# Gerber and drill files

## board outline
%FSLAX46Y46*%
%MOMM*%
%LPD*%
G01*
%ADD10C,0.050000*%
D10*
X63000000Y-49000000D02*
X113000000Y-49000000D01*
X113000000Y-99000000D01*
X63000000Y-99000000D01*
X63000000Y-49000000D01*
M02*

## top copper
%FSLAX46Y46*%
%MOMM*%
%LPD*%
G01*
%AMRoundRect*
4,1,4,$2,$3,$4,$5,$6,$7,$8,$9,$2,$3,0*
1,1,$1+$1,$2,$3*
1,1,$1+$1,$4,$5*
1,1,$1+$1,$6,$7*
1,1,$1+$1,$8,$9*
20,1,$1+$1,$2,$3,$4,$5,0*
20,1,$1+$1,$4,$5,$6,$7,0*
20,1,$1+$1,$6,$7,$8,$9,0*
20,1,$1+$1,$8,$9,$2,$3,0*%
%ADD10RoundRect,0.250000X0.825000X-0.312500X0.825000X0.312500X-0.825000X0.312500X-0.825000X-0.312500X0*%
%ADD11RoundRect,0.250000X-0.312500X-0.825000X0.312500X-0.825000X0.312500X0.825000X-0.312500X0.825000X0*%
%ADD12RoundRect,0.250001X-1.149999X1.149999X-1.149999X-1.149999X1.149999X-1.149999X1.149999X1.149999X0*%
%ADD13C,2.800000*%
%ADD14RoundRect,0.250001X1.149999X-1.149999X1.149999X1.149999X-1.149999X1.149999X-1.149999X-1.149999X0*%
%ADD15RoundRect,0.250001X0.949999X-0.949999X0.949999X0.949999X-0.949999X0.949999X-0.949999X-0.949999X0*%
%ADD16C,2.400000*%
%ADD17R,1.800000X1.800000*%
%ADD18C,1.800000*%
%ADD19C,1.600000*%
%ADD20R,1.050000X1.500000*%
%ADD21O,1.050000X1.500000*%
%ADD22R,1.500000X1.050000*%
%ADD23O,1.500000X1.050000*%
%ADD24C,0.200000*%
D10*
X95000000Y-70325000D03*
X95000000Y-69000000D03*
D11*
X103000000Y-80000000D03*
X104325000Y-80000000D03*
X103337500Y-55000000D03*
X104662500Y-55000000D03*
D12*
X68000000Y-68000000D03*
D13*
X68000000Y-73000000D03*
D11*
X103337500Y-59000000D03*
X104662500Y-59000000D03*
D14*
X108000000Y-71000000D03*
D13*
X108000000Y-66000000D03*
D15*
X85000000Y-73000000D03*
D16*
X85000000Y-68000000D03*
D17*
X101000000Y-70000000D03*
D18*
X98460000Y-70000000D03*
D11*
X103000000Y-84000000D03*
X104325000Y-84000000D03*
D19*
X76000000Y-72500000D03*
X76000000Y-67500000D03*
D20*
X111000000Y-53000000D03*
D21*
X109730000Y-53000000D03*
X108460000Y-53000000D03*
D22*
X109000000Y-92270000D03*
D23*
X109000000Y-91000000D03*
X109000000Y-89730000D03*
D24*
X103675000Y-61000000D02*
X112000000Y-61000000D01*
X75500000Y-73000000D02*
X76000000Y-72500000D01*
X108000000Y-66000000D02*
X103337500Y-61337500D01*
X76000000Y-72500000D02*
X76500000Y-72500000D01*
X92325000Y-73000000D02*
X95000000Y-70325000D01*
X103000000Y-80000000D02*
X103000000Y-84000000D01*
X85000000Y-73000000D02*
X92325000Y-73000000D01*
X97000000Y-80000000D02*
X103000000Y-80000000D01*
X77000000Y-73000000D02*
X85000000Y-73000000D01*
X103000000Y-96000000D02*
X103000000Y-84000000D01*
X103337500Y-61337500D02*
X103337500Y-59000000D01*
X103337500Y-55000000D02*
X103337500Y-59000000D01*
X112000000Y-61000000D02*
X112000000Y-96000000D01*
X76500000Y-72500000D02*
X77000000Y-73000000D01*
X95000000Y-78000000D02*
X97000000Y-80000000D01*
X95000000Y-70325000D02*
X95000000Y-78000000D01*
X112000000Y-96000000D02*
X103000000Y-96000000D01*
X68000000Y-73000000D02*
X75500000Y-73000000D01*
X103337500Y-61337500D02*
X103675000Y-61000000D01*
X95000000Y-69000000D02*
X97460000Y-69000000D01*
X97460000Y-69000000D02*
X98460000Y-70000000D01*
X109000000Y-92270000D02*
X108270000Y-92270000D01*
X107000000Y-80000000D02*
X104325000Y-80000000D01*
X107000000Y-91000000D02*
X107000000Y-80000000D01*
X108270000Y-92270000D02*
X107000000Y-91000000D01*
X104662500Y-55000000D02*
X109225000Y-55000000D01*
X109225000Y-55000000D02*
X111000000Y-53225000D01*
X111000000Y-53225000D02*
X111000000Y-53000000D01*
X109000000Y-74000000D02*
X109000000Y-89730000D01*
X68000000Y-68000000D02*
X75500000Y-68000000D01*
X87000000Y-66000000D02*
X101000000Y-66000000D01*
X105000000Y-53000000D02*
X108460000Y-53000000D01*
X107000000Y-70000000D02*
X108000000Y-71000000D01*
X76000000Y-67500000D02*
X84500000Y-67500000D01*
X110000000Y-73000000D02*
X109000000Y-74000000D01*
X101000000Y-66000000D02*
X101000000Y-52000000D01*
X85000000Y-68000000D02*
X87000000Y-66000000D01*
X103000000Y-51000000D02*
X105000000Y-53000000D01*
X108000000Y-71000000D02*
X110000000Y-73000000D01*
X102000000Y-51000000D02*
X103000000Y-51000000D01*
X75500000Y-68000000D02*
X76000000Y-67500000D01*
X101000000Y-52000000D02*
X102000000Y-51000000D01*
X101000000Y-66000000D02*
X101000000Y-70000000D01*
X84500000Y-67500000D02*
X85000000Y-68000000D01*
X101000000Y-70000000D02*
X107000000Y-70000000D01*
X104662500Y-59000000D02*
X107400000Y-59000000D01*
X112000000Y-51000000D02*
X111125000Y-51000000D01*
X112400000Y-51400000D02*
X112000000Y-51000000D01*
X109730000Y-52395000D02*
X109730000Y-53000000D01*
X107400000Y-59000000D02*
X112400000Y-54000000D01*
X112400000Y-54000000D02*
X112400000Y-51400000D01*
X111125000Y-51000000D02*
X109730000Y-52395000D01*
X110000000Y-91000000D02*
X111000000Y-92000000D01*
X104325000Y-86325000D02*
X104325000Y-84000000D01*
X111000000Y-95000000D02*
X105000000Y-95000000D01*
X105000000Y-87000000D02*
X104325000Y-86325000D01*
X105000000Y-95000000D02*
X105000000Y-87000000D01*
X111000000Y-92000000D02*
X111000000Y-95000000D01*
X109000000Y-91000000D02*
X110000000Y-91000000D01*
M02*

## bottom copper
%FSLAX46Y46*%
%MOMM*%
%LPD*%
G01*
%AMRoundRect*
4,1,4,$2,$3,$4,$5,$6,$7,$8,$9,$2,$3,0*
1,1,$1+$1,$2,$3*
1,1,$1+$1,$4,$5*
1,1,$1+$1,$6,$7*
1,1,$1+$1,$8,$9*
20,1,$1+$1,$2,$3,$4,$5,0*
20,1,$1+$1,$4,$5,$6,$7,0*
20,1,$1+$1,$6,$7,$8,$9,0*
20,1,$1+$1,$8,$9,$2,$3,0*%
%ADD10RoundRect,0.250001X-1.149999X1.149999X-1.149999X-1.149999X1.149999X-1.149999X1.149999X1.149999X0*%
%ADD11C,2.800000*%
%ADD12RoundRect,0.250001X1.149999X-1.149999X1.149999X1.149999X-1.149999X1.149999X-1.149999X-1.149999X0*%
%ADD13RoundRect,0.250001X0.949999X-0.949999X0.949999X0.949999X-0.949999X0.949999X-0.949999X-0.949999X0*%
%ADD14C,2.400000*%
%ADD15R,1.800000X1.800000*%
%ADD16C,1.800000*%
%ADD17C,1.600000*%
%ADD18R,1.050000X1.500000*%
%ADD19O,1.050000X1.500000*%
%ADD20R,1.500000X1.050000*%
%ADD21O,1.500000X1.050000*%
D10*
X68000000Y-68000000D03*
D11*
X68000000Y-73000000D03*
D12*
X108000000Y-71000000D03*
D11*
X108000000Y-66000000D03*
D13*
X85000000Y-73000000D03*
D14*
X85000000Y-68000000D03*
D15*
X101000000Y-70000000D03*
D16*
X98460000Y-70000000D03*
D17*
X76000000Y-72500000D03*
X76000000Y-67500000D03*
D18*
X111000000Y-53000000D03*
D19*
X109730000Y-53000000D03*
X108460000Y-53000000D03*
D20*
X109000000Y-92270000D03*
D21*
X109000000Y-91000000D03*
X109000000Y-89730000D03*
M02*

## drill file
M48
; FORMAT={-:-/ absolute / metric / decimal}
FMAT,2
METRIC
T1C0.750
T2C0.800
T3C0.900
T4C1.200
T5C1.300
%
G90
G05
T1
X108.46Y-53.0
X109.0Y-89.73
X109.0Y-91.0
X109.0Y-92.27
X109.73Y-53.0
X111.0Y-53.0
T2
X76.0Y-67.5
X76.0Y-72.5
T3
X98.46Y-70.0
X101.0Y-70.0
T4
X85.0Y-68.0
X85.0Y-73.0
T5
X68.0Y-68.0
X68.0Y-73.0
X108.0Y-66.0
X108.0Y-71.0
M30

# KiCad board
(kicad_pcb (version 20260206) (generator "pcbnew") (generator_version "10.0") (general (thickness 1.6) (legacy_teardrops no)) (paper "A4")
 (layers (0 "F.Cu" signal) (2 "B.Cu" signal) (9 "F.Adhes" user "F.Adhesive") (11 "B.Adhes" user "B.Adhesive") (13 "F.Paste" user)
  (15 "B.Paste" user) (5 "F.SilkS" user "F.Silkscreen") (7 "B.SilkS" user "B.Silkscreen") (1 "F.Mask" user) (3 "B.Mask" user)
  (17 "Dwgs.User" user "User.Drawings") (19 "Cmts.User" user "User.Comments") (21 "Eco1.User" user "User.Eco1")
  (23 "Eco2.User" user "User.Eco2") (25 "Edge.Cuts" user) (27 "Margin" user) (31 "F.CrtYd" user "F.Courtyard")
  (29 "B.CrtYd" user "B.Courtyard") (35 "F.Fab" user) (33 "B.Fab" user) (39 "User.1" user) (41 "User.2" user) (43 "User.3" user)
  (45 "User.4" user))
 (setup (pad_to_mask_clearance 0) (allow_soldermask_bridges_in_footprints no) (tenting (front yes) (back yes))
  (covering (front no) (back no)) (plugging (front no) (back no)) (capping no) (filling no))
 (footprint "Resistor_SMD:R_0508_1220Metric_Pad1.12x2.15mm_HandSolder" (layer "F.Cu") (at 95 69.6625 90)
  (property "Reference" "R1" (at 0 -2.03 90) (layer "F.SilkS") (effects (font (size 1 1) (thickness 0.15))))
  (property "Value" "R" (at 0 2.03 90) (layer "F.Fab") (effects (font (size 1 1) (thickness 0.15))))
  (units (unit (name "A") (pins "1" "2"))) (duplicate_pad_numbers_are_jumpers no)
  (pad "1" smd roundrect (at -0.6625 0 90) (size 1.125 2.15) (layers "F.Cu" "F.Mask" "F.Paste") (roundrect_rratio 0.222222) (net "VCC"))
  (pad "2" smd roundrect (at 0.6625 0 90) (size 1.125 2.15) (layers "F.Cu" "F.Mask" "F.Paste") (roundrect_rratio 0.222222)
   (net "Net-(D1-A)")))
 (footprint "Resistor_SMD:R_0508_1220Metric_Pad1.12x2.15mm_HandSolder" (layer "F.Cu") (at 103.6625 80)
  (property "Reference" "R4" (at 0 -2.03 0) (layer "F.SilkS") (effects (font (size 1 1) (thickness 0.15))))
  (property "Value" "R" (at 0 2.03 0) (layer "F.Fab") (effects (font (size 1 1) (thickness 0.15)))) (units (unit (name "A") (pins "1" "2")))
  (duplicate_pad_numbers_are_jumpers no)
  (pad "1" smd roundrect (at -0.6625 0) (size 1.125 2.15) (layers "F.Cu" "F.Mask" "F.Paste") (roundrect_rratio 0.222222) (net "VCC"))
  (pad "2" smd roundrect (at 0.6625 0) (size 1.125 2.15) (layers "F.Cu" "F.Mask" "F.Paste") (roundrect_rratio 0.222222) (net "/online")))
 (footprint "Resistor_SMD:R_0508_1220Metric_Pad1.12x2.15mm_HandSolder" (layer "F.Cu") (at 104 55)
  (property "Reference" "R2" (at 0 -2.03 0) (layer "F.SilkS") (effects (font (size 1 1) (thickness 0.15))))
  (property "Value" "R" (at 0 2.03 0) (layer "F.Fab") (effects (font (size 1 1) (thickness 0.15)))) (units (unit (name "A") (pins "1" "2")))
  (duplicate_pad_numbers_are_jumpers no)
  (pad "1" smd roundrect (at -0.6625 0) (size 1.125 2.15) (layers "F.Cu" "F.Mask" "F.Paste") (roundrect_rratio 0.222222) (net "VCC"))
  (pad "2" smd roundrect (at 0.6625 0) (size 1.125 2.15) (layers "F.Cu" "F.Mask" "F.Paste") (roundrect_rratio 0.222222) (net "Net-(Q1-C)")))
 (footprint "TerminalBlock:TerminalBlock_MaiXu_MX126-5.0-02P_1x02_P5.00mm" (layer "F.Cu") (at 68 68 -90)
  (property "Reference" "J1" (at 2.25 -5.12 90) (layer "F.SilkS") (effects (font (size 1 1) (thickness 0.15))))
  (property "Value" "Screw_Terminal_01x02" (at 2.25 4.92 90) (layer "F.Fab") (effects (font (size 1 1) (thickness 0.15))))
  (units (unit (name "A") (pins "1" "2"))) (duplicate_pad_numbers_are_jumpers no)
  (pad "1" thru_hole roundrect (at 0 0 270) (size 2.8 2.8) (drill 1.3) (layers "*.Cu" "*.Mask") (remove_unused_layers no)
   (roundrect_rratio 0.089286) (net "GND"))
  (pad "2" thru_hole circle (at 5 0 270) (size 2.8 2.8) (drill 1.3) (layers "*.Cu" "*.Mask") (remove_unused_layers no) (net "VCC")))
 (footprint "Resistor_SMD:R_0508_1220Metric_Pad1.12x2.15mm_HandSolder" (layer "F.Cu") (at 104 59)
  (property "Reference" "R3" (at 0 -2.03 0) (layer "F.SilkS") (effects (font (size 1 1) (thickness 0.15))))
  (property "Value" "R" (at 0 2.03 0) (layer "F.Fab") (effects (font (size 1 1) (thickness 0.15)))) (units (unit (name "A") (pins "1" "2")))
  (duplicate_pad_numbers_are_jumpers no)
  (pad "1" smd roundrect (at -0.6625 0) (size 1.125 2.15) (layers "F.Cu" "F.Mask" "F.Paste") (roundrect_rratio 0.222222) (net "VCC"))
  (pad "2" smd roundrect (at 0.6625 0) (size 1.125 2.15) (layers "F.Cu" "F.Mask" "F.Paste") (roundrect_rratio 0.222222) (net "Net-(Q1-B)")))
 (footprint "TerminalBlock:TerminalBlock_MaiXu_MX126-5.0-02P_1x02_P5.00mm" (layer "F.Cu") (at 108 71 90)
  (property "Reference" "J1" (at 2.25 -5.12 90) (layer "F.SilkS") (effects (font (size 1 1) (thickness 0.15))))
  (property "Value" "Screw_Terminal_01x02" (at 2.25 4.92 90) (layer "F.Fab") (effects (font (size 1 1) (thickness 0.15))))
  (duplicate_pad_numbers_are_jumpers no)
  (pad "1" thru_hole roundrect (at 0 0 90) (size 2.8 2.8) (drill 1.3) (layers "*.Cu" "*.Mask") (remove_unused_layers no)
   (roundrect_rratio 0.089286) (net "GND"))
  (pad "2" thru_hole circle (at 5 0 90) (size 2.8 2.8) (drill 1.3) (layers "*.Cu" "*.Mask") (remove_unused_layers no) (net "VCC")))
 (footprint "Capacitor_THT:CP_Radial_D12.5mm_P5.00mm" (layer "F.Cu") (at 85 73 90)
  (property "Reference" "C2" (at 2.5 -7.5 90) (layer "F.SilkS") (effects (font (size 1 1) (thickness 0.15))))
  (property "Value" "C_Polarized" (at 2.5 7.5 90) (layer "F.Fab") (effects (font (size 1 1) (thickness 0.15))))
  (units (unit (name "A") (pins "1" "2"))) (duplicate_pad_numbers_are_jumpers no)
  (pad "1" thru_hole roundrect (at 0 0 90) (size 2.4 2.4) (drill 1.2) (layers "*.Cu" "*.Mask") (remove_unused_layers no)
   (roundrect_rratio 0.104167) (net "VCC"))
  (pad "2" thru_hole circle (at 5 0 90) (size 2.4 2.4) (drill 1.2) (layers "*.Cu" "*.Mask") (remove_unused_layers no) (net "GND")))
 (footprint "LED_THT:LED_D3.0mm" (layer "F.Cu") (at 101 70 180)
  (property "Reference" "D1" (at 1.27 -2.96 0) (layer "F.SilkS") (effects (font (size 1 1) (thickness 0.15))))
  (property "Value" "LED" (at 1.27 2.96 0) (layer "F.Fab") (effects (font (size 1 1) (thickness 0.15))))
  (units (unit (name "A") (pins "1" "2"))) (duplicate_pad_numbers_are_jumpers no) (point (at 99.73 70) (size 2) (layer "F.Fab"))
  (pad "1" thru_hole rect (at 0 0 180) (size 1.8 1.8) (drill 0.9) (layers "*.Cu" "*.Mask") (remove_unused_layers no) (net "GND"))
  (pad "2" thru_hole circle (at 2.54 0 180) (size 1.8 1.8) (drill 0.9) (layers "*.Cu" "*.Mask") (remove_unused_layers no) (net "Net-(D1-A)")))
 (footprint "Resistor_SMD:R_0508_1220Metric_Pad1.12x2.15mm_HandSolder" (layer "F.Cu") (at 103.6625 84)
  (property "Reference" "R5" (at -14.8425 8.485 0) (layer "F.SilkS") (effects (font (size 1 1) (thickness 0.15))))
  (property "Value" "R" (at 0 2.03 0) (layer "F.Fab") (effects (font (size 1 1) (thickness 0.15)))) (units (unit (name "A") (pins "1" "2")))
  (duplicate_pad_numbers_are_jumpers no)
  (pad "1" smd roundrect (at -0.6625 0) (size 1.125 2.15) (layers "F.Cu" "F.Mask" "F.Paste") (roundrect_rratio 0.222222) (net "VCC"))
  (pad "2" smd roundrect (at 0.6625 0) (size 1.125 2.15) (layers "F.Cu" "F.Mask" "F.Paste") (roundrect_rratio 0.222222) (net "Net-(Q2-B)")))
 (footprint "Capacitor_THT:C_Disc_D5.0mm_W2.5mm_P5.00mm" (layer "F.Cu") (at 76 72.5 90)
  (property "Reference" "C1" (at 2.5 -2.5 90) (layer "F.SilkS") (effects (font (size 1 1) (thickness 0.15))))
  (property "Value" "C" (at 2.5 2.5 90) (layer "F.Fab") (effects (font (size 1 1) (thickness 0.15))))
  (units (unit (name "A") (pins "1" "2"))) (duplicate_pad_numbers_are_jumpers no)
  (pad "1" thru_hole circle (at 0 0 90) (size 1.6 1.6) (drill 0.8) (layers "*.Cu" "*.Mask") (remove_unused_layers no) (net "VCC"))
  (pad "2" thru_hole circle (at 5 0 90) (size 1.6 1.6) (drill 0.8) (layers "*.Cu" "*.Mask") (remove_unused_layers no) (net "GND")))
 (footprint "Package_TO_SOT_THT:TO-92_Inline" (layer "F.Cu") (at 111 53 180)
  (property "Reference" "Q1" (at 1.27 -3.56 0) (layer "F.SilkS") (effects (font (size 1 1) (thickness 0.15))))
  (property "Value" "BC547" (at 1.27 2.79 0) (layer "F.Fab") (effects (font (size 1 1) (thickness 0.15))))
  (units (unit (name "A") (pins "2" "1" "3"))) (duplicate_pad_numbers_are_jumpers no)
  (pad "1" thru_hole rect (at 0 0 180) (size 1.05 1.5) (drill 0.75) (layers "*.Cu" "*.Mask") (remove_unused_layers no) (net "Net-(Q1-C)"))
  (pad "2" thru_hole oval (at 1.27 0 180) (size 1.05 1.5) (drill 0.75) (layers "*.Cu" "*.Mask") (remove_unused_layers no) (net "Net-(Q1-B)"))
  (pad "3" thru_hole oval (at 2.54 0 180) (size 1.05 1.5) (drill 0.75) (layers "*.Cu" "*.Mask") (remove_unused_layers no) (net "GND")))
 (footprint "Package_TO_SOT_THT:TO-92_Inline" (layer "F.Cu") (at 109 92.27 90)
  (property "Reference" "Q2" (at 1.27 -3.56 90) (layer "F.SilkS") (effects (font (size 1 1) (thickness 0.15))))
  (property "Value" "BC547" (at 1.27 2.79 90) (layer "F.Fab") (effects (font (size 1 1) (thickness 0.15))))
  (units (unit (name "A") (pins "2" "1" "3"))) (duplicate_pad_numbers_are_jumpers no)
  (pad "1" thru_hole rect (at 0 0 90) (size 1.05 1.5) (drill 0.75) (layers "*.Cu" "*.Mask") (remove_unused_layers no) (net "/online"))
  (pad "2" thru_hole oval (at 1.27 0 90) (size 1.05 1.5) (drill 0.75) (layers "*.Cu" "*.Mask") (remove_unused_layers no) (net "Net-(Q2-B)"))
  (pad "3" thru_hole oval (at 2.54 0 90) (size 1.05 1.5) (drill 0.75) (layers "*.Cu" "*.Mask") (remove_unused_layers no) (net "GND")))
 (gr_rect (start 63 49) (end 113 99) (stroke (width 0.05) (type default)) (fill no) (layer "Edge.Cuts"))
 (segment (start 103.675 61) (end 112 61) (width 0.2) (layer "F.Cu") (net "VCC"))
 (segment (start 75.5 73) (end 76 72.5) (width 0.2) (layer "F.Cu") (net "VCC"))
 (segment (start 108 66) (end 103.3375 61.3375) (width 0.2) (layer "F.Cu") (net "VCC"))
 (segment (start 76 72.5) (end 76.5 72.5) (width 0.2) (layer "F.Cu") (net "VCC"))
 (segment (start 92.325 73) (end 95 70.325) (width 0.2) (layer "F.Cu") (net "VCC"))
 (segment (start 103 80) (end 103 84) (width 0.2) (layer "F.Cu") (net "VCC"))
 (segment (start 85 73) (end 92.325 73) (width 0.2) (layer "F.Cu") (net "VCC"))
 (segment (start 97 80) (end 103 80) (width 0.2) (layer "F.Cu") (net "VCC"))
 (segment (start 77 73) (end 85 73) (width 0.2) (layer "F.Cu") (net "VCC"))
 (segment (start 103 96) (end 103 84) (width 0.2) (layer "F.Cu") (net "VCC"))
 (segment (start 103.3375 61.3375) (end 103.3375 59) (width 0.2) (layer "F.Cu") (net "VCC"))
 (segment (start 103.3375 55) (end 103.3375 59) (width 0.2) (layer "F.Cu") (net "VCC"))
 (segment (start 112 61) (end 112 96) (width 0.2) (layer "F.Cu") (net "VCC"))
 (segment (start 76.5 72.5) (end 77 73) (width 0.2) (layer "F.Cu") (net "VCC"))
 (segment (start 95 78) (end 97 80) (width 0.2) (layer "F.Cu") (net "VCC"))
 (segment (start 95 70.325) (end 95 78) (width 0.2) (layer "F.Cu") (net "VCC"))
 (segment (start 112 96) (end 103 96) (width 0.2) (layer "F.Cu") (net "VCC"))
 (segment (start 68 73) (end 75.5 73) (width 0.2) (layer "F.Cu") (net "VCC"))
 (segment (start 103.3375 61.3375) (end 103.675 61) (width 0.2) (layer "F.Cu") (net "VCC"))
 (segment (start 95 69) (end 97.46 69) (width 0.2) (layer "F.Cu") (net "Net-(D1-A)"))
 (segment (start 97.46 69) (end 98.46 70) (width 0.2) (layer "F.Cu") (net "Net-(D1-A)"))
 (segment (start 109 92.27) (end 108.27 92.27) (width 0.2) (layer "F.Cu") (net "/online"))
 (segment (start 107 80) (end 104.325 80) (width 0.2) (layer "F.Cu") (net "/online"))
 (segment (start 107 91) (end 107 80) (width 0.2) (layer "F.Cu") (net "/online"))
 (segment (start 108.27 92.27) (end 107 91) (width 0.2) (layer "F.Cu") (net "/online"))
 (segment (start 104.6625 55) (end 109.225 55) (width 0.2) (layer "F.Cu") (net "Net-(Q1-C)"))
 (segment (start 109.225 55) (end 111 53.225) (width 0.2) (layer "F.Cu") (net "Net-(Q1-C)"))
 (segment (start 111 53.225) (end 111 53) (width 0.2) (layer "F.Cu") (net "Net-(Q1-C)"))
 (segment (start 109 74) (end 109 89.73) (width 0.2) (layer "F.Cu") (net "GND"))
 (segment (start 68 68) (end 75.5 68) (width 0.2) (layer "F.Cu") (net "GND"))
 (segment (start 87 66) (end 101 66) (width 0.2) (layer "F.Cu") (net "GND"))
 (segment (start 105 53) (end 108.46 53) (width 0.2) (layer "F.Cu") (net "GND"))
 (segment (start 107 70) (end 108 71) (width 0.2) (layer "F.Cu") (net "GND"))
 (segment (start 76 67.5) (end 84.5 67.5) (width 0.2) (layer "F.Cu") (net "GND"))
 (segment (start 110 73) (end 109 74) (width 0.2) (layer "F.Cu") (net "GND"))
 (segment (start 101 66) (end 101 52) (width 0.2) (layer "F.Cu") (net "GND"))
 (segment (start 85 68) (end 87 66) (width 0.2) (layer "F.Cu") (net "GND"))
 (segment (start 103 51) (end 105 53) (width 0.2) (layer "F.Cu") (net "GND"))
 (segment (start 108 71) (end 110 73) (width 0.2) (layer "F.Cu") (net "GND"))
 (segment (start 102 51) (end 103 51) (width 0.2) (layer "F.Cu") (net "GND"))
 (segment (start 75.5 68) (end 76 67.5) (width 0.2) (layer "F.Cu") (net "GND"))
 (segment (start 101 52) (end 102 51) (width 0.2) (layer "F.Cu") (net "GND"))
 (segment (start 101 66) (end 101 70) (width 0.2) (layer "F.Cu") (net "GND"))
 (segment (start 84.5 67.5) (end 85 68) (width 0.2) (layer "F.Cu") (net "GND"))
 (segment (start 101 70) (end 107 70) (width 0.2) (layer "F.Cu") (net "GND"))
 (segment (start 104.6625 59) (end 107.4 59) (width 0.2) (layer "F.Cu") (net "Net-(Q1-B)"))
 (segment (start 112 51) (end 111.125 51) (width 0.2) (layer "F.Cu") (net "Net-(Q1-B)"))
 (segment (start 112.4 51.4) (end 112 51) (width 0.2) (layer "F.Cu") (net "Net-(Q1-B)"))
 (segment (start 109.73 52.395) (end 109.73 53) (width 0.2) (layer "F.Cu") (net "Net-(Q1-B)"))
 (segment (start 107.4 59) (end 112.4 54) (width 0.2) (layer "F.Cu") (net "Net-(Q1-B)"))
 (segment (start 112.4 54) (end 112.4 51.4) (width 0.2) (layer "F.Cu") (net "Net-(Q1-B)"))
 (segment (start 111.125 51) (end 109.73 52.395) (width 0.2) (layer "F.Cu") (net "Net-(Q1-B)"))
 (segment (start 110 91) (end 111 92) (width 0.2) (layer "F.Cu") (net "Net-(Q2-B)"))
 (segment (start 104.325 86.325) (end 104.325 84) (width 0.2) (layer "F.Cu") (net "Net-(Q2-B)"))
 (segment (start 111 95) (end 105 95) (width 0.2) (layer "F.Cu") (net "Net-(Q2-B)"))
 (segment (start 105 87) (end 104.325 86.325) (width 0.2) (layer "F.Cu") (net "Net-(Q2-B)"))
 (segment (start 105 95) (end 105 87) (width 0.2) (layer "F.Cu") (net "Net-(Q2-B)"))
 (segment (start 111 92) (end 111 95) (width 0.2) (layer "F.Cu") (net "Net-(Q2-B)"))
 (segment (start 109 91) (end 110 91) (width 0.2) (layer "F.Cu") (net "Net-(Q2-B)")))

